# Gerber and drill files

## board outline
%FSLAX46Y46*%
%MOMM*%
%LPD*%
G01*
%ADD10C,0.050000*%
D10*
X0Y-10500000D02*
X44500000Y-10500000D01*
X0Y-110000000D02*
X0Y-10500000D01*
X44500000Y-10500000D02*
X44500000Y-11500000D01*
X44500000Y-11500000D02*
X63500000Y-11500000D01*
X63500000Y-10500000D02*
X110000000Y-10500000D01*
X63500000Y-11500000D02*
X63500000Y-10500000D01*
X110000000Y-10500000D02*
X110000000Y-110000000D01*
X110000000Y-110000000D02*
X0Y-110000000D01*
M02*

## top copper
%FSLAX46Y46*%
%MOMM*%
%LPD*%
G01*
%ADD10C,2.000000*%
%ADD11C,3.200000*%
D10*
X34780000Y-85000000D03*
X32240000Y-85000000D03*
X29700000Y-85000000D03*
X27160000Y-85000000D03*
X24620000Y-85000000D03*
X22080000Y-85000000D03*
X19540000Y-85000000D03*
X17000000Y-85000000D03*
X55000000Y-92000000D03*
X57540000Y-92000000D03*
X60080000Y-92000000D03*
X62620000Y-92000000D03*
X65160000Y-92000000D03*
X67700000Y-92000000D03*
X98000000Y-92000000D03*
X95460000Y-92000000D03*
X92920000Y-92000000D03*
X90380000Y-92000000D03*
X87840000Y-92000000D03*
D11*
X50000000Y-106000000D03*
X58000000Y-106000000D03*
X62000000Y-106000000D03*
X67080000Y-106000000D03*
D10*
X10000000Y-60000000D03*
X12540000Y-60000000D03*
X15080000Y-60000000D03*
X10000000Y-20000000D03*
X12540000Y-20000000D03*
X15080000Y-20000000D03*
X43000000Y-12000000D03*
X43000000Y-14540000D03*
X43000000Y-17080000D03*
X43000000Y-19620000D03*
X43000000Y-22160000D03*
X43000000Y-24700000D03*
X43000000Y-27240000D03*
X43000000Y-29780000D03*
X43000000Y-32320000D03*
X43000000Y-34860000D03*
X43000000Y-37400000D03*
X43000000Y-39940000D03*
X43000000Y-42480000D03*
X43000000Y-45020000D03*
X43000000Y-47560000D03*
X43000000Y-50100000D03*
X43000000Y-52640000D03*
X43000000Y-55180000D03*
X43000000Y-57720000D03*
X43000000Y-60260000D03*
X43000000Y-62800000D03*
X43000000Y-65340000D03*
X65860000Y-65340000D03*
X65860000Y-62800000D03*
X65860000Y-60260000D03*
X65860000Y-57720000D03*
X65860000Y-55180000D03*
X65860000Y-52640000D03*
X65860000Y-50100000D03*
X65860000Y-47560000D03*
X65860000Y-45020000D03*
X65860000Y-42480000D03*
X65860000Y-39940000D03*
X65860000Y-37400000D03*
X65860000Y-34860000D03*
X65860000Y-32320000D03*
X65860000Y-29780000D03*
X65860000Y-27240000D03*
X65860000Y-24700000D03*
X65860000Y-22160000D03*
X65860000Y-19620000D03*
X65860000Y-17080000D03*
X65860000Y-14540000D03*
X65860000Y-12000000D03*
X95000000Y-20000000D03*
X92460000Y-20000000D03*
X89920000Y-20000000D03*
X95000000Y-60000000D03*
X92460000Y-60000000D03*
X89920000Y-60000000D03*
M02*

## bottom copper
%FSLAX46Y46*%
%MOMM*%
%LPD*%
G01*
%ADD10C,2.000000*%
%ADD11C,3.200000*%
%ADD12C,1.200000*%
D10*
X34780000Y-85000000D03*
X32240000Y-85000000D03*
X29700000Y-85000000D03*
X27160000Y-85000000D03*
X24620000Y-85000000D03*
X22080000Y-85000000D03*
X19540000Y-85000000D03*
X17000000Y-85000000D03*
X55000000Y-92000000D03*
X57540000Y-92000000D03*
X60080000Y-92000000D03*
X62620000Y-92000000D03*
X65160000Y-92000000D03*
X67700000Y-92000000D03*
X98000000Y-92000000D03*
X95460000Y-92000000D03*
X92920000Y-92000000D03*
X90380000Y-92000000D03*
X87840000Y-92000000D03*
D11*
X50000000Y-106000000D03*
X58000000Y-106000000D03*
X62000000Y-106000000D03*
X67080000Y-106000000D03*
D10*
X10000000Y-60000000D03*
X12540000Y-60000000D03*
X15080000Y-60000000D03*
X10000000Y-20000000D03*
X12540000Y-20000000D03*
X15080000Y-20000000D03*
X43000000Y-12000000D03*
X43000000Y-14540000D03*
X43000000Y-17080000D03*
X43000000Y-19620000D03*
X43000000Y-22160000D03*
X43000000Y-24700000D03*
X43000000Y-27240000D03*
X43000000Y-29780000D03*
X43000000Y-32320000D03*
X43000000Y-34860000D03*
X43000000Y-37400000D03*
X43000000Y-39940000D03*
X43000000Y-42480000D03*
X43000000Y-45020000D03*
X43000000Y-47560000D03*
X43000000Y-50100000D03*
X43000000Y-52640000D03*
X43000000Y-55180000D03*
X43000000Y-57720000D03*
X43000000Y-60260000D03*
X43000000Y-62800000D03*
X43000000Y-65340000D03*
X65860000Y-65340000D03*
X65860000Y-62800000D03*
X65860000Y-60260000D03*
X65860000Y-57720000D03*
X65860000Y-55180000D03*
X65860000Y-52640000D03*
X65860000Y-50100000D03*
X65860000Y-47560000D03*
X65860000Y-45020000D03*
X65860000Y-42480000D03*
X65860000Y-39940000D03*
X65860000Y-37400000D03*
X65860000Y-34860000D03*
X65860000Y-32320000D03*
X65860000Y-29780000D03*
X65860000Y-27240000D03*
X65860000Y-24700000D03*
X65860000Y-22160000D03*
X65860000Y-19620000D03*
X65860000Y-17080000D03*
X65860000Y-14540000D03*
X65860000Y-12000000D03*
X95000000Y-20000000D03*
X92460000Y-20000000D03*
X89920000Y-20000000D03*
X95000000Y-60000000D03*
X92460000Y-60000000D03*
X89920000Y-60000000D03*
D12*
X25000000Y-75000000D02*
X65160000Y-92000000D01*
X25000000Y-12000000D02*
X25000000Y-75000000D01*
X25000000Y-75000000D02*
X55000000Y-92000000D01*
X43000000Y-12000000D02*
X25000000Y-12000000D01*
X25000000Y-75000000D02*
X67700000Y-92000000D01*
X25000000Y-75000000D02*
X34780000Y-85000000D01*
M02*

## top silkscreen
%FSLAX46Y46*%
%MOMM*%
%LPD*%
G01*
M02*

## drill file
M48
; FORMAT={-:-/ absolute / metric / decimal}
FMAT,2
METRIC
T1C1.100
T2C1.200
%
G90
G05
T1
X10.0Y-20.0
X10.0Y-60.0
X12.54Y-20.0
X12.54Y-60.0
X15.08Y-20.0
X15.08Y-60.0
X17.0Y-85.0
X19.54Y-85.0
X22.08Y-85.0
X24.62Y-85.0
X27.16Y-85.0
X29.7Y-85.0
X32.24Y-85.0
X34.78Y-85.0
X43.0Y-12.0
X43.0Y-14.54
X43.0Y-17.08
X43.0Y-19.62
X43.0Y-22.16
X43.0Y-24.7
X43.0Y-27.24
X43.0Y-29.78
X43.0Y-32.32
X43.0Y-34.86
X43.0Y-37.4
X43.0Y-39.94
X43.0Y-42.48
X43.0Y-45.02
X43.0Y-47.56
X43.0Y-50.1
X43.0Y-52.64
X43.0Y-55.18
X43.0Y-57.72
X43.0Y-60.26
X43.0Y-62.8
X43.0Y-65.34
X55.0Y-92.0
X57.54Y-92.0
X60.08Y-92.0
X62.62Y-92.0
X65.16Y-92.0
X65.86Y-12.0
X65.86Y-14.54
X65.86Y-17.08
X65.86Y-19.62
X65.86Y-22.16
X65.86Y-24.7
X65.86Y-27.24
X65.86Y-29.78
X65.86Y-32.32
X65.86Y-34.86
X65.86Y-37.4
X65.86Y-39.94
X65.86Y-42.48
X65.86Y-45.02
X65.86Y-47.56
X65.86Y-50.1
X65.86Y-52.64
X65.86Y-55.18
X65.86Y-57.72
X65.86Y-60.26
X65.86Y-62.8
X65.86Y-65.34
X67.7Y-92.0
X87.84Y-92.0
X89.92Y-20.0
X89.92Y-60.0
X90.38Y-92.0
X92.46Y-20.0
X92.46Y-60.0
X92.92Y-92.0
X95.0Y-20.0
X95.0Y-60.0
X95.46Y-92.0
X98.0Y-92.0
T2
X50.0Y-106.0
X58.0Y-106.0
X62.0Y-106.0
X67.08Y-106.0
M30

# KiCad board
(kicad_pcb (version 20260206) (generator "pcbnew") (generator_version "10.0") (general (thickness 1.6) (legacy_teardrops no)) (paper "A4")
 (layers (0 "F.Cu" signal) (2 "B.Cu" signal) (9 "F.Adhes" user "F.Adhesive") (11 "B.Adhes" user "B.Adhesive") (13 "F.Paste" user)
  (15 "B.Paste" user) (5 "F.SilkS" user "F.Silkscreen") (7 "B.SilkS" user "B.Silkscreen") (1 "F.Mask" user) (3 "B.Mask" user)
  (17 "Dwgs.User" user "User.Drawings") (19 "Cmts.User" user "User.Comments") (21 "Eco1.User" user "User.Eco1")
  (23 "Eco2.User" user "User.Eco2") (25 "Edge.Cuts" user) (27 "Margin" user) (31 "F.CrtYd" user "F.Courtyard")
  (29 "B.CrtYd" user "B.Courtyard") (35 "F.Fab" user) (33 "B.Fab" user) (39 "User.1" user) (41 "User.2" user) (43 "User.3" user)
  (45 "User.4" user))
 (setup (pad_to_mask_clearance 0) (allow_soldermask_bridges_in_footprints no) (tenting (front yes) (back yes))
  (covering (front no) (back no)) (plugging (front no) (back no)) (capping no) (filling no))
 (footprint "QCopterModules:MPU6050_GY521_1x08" (layer "F.Cu") (at 34.78 85 -90)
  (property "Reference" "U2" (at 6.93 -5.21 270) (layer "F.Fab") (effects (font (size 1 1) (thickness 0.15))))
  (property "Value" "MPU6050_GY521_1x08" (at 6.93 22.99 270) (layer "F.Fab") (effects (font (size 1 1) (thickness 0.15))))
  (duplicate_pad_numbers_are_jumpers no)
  (pad "1" thru_hole circle (at 0 0 270) (size 2 2) (drill 1.1) (layers "*.Cu" "*.Mask") (remove_unused_layers no) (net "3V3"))
  (pad "2" thru_hole circle (at 0 2.54 270) (size 2 2) (drill 1.1) (layers "*.Cu" "*.Mask") (remove_unused_layers no) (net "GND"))
  (pad "3" thru_hole circle (at 0 5.08 270) (size 2 2) (drill 1.1) (layers "*.Cu" "*.Mask") (remove_unused_layers no) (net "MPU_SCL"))
  (pad "4" thru_hole circle (at 0 7.62 270) (size 2 2) (drill 1.1) (layers "*.Cu" "*.Mask") (remove_unused_layers no) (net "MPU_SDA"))
  (pad "5" thru_hole circle (at 0 10.16 270) (size 2 2) (drill 1.1) (layers "*.Cu" "*.Mask") (remove_unused_layers no)
   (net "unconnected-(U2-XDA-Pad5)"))
  (pad "6" thru_hole circle (at 0 12.7 270) (size 2 2) (drill 1.1) (layers "*.Cu" "*.Mask") (remove_unused_layers no)
   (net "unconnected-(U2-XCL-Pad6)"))
  (pad "7" thru_hole circle (at 0 15.24 270) (size 2 2) (drill 1.1) (layers "*.Cu" "*.Mask") (remove_unused_layers no) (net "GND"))
  (pad "8" thru_hole circle (at 0 17.78 270) (size 2 2) (drill 1.1) (layers "*.Cu" "*.Mask") (remove_unused_layers no) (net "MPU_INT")))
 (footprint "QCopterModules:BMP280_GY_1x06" (layer "F.Cu") (at 55 92 90)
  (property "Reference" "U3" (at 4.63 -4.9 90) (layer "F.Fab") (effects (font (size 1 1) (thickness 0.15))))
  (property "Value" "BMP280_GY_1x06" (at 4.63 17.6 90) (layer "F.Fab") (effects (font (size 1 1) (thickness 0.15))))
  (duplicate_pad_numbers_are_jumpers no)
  (pad "1" thru_hole circle (at 0 0 90) (size 2 2) (drill 1.1) (layers "*.Cu" "*.Mask") (remove_unused_layers no) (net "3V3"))
  (pad "2" thru_hole circle (at 0 2.54 90) (size 2 2) (drill 1.1) (layers "*.Cu" "*.Mask") (remove_unused_layers no) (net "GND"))
  (pad "3" thru_hole circle (at 0 5.08 90) (size 2 2) (drill 1.1) (layers "*.Cu" "*.Mask") (remove_unused_layers no) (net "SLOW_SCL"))
  (pad "4" thru_hole circle (at 0 7.62 90) (size 2 2) (drill 1.1) (layers "*.Cu" "*.Mask") (remove_unused_layers no) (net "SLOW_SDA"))
  (pad "5" thru_hole circle (at 0 10.16 90) (size 2 2) (drill 1.1) (layers "*.Cu" "*.Mask") (remove_unused_layers no) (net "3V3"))
  (pad "6" thru_hole circle (at 0 12.7 90) (size 2 2) (drill 1.1) (layers "*.Cu" "*.Mask") (remove_unused_layers no) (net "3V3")))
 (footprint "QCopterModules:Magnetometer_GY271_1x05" (layer "F.Cu") (at 98 92 -90)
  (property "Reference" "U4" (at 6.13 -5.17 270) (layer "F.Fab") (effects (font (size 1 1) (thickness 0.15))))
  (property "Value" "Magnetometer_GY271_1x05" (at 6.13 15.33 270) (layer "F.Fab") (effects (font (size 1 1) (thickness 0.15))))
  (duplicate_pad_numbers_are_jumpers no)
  (pad "1" thru_hole circle (at 0 0 270) (size 2 2) (drill 1.1) (layers "*.Cu" "*.Mask") (remove_unused_layers no) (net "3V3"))
  (pad "2" thru_hole circle (at 0 2.54 270) (size 2 2) (drill 1.1) (layers "*.Cu" "*.Mask") (remove_unused_layers no) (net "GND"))
  (pad "3" thru_hole circle (at 0 5.08 270) (size 2 2) (drill 1.1) (layers "*.Cu" "*.Mask") (remove_unused_layers no) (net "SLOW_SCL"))
  (pad "4" thru_hole circle (at 0 7.62 270) (size 2 2) (drill 1.1) (layers "*.Cu" "*.Mask") (remove_unused_layers no) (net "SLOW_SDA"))
  (pad "5" thru_hole circle (at 0 10.16 270) (size 2 2) (drill 1.1) (layers "*.Cu" "*.Mask") (remove_unused_layers no) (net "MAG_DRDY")))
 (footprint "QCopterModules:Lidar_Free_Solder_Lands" (layer "F.Cu") (at 50 106)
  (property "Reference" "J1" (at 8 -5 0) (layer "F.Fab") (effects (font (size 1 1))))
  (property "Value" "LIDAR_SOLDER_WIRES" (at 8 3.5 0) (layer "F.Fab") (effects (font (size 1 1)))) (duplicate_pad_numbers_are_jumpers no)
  (pad "1" thru_hole circle (at 0 0) (size 3.2 3.2) (drill 1.2) (layers "*.Cu" "*.Mask") (remove_unused_layers no) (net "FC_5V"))
  (pad "2" thru_hole circle (at 8 0) (size 3.2 3.2) (drill 1.2) (layers "*.Cu" "*.Mask") (remove_unused_layers no) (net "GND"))
  (pad "3" thru_hole circle (at 12 0) (size 3.2 3.2) (drill 1.2) (layers "*.Cu" "*.Mask") (remove_unused_layers no) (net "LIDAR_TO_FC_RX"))
  (pad "4" thru_hole circle (at 17.08 0) (size 3.2 3.2) (drill 1.2) (layers "*.Cu" "*.Mask") (remove_unused_layers no)
   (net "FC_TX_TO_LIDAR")))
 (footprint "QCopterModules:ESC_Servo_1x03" (layer "F.Cu") (at 10 60 90)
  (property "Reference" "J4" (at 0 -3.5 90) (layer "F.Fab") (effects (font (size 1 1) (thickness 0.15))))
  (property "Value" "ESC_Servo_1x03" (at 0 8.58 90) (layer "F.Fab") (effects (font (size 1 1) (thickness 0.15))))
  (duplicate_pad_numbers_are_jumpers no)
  (pad "1" thru_hole circle (at 0 0 90) (size 2 2) (drill 1.1) (layers "*.Cu" "*.Mask") (remove_unused_layers no) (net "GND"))
  (pad "2" thru_hole circle (at 0 2.54 90) (size 2 2) (drill 1.1) (layers "*.Cu" "*.Mask") (remove_unused_layers no) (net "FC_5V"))
  (pad "3" thru_hole circle (at 0 5.08 90) (size 2 2) (drill 1.1) (layers "*.Cu" "*.Mask") (remove_unused_layers no) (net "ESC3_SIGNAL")))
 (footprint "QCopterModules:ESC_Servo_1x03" (layer "F.Cu") (at 10 20 90)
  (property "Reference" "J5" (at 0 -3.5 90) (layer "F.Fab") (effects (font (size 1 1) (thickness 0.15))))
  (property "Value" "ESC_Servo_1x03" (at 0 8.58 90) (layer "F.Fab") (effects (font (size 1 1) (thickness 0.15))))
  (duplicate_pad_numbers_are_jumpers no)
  (pad "1" thru_hole circle (at 0 0 90) (size 2 2) (drill 1.1) (layers "*.Cu" "*.Mask") (remove_unused_layers no) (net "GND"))
  (pad "2" thru_hole circle (at 0 2.54 90) (size 2 2) (drill 1.1) (layers "*.Cu" "*.Mask") (remove_unused_layers no)
   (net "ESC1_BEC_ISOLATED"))
  (pad "3" thru_hole circle (at 0 5.08 90) (size 2 2) (drill 1.1) (layers "*.Cu" "*.Mask") (remove_unused_layers no) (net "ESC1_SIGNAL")))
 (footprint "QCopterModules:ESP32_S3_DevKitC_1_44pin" (layer "F.Cu") (at 43 12)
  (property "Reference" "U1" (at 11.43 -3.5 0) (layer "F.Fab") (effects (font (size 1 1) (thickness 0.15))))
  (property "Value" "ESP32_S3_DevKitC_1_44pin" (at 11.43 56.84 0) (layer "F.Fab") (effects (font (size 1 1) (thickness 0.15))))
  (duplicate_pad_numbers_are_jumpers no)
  (pad "1" thru_hole circle (at 0 0) (size 2 2) (drill 1.1) (layers "*.Cu" "*.Mask") (remove_unused_layers no) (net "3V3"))
  (pad "2" thru_hole circle (at 0 2.54) (size 2 2) (drill 1.1) (layers "*.Cu" "*.Mask") (remove_unused_layers no))
  (pad "3" thru_hole circle (at 0 5.08) (size 2 2) (drill 1.1) (layers "*.Cu" "*.Mask") (remove_unused_layers no)
   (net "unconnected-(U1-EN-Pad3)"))
  (pad "4" thru_hole circle (at 0 7.62) (size 2 2) (drill 1.1) (layers "*.Cu" "*.Mask") (remove_unused_layers no) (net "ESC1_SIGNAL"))
  (pad "5" thru_hole circle (at 0 10.16) (size 2 2) (drill 1.1) (layers "*.Cu" "*.Mask") (remove_unused_layers no)
   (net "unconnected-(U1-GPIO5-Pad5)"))
  (pad "6" thru_hole circle (at 0 12.7) (size 2 2) (drill 1.1) (layers "*.Cu" "*.Mask") (remove_unused_layers no)
   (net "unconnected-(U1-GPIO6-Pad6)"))
  (pad "7" thru_hole circle (at 0 15.24) (size 2 2) (drill 1.1) (layers "*.Cu" "*.Mask") (remove_unused_layers no)
   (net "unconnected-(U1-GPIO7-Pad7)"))
  (pad "8" thru_hole circle (at 0 17.78) (size 2 2) (drill 1.1) (layers "*.Cu" "*.Mask") (remove_unused_layers no) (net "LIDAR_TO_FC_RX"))
  (pad "9" thru_hole circle (at 0 20.32) (size 2 2) (drill 1.1) (layers "*.Cu" "*.Mask") (remove_unused_layers no) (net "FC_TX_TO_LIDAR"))
  (pad "10" thru_hole circle (at 0 22.86) (size 2 2) (drill 1.1) (layers "*.Cu" "*.Mask") (remove_unused_layers no)
   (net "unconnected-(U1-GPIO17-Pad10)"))
  (pad "11" thru_hole circle (at 0 25.4) (size 2 2) (drill 1.1) (layers "*.Cu" "*.Mask") (remove_unused_layers no) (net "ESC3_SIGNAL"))
  (pad "12" thru_hole circle (at 0 27.94) (size 2 2) (drill 1.1) (layers "*.Cu" "*.Mask") (remove_unused_layers no)
   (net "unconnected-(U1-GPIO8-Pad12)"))
  (pad "13" thru_hole circle (at 0 30.48) (size 2 2) (drill 1.1) (layers "*.Cu" "*.Mask") (remove_unused_layers no)
   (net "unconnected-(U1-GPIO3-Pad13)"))
  (pad "14" thru_hole circle (at 0 33.02) (size 2 2) (drill 1.1) (layers "*.Cu" "*.Mask") (remove_unused_layers no)
   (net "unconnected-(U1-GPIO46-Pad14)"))
  (pad "15" thru_hole circle (at 0 35.56) (size 2 2) (drill 1.1) (layers "*.Cu" "*.Mask") (remove_unused_layers no)
   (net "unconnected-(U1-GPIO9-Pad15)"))
  (pad "16" thru_hole circle (at 0 38.1) (size 2 2) (drill 1.1) (layers "*.Cu" "*.Mask") (remove_unused_layers no)
   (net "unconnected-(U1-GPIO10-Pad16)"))
  (pad "17" thru_hole circle (at 0 40.64) (size 2 2) (drill 1.1) (layers "*.Cu" "*.Mask") (remove_unused_layers no)
   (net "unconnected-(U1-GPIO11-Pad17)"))
  (pad "18" thru_hole circle (at 0 43.18) (size 2 2) (drill 1.1) (layers "*.Cu" "*.Mask") (remove_unused_layers no) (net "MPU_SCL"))
  (pad "19" thru_hole circle (at 0 45.72) (size 2 2) (drill 1.1) (layers "*.Cu" "*.Mask") (remove_unused_layers no) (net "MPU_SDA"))
  (pad "20" thru_hole circle (at 0 48.26) (size 2 2) (drill 1.1) (layers "*.Cu" "*.Mask") (remove_unused_layers no) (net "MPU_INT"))
  (pad "21" thru_hole circle (at 0 50.8) (size 2 2) (drill 1.1) (layers "*.Cu" "*.Mask") (remove_unused_layers no) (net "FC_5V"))
  (pad "22" thru_hole circle (at 0 53.34) (size 2 2) (drill 1.1) (layers "*.Cu" "*.Mask") (remove_unused_layers no) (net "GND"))
  (pad "23" thru_hole circle (at 22.86 53.34) (size 2 2) (drill 1.1) (layers "*.Cu" "*.Mask") (remove_unused_layers no) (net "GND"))
  (pad "24" thru_hole circle (at 22.86 50.8) (size 2 2) (drill 1.1) (layers "*.Cu" "*.Mask") (remove_unused_layers no) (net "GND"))
  (pad "25" thru_hole circle (at 22.86 48.26) (size 2 2) (drill 1.1) (layers "*.Cu" "*.Mask") (remove_unused_layers no)
   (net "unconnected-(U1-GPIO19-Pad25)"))
  (pad "26" thru_hole circle (at 22.86 45.72) (size 2 2) (drill 1.1) (layers "*.Cu" "*.Mask") (remove_unused_layers no)
   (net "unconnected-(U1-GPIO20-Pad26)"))
  (pad "27" thru_hole circle (at 22.86 43.18) (size 2 2) (drill 1.1) (layers "*.Cu" "*.Mask") (remove_unused_layers no) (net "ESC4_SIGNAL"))
  (pad "28" thru_hole circle (at 22.86 40.64) (size 2 2) (drill 1.1) (layers "*.Cu" "*.Mask") (remove_unused_layers no)
   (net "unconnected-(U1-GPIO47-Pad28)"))
  (pad "29" thru_hole circle (at 22.86 38.1) (size 2 2) (drill 1.1) (layers "*.Cu" "*.Mask") (remove_unused_layers no)
   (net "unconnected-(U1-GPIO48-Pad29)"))
  (pad "30" thru_hole circle (at 22.86 35.56) (size 2 2) (drill 1.1) (layers "*.Cu" "*.Mask") (remove_unused_layers no)
   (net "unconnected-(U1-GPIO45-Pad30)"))
  (pad "31" thru_hole circle (at 22.86 33.02) (size 2 2) (drill 1.1) (layers "*.Cu" "*.Mask") (remove_unused_layers no)
   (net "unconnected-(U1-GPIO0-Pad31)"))
  (pad "32" thru_hole circle (at 22.86 30.48) (size 2 2) (drill 1.1) (layers "*.Cu" "*.Mask") (remove_unused_layers no)
   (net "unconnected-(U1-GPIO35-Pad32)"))
  (pad "33" thru_hole circle (at 22.86 27.94) (size 2 2) (drill 1.1) (layers "*.Cu" "*.Mask") (remove_unused_layers no)
   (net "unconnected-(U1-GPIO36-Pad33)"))
  (pad "34" thru_hole circle (at 22.86 25.4) (size 2 2) (drill 1.1) (layers "*.Cu" "*.Mask") (remove_unused_layers no)
   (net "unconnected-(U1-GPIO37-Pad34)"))
  (pad "35" thru_hole circle (at 22.86 22.86) (size 2 2) (drill 1.1) (layers "*.Cu" "*.Mask") (remove_unused_layers no)
   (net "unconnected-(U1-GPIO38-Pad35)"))
  (pad "36" thru_hole circle (at 22.86 20.32) (size 2 2) (drill 1.1) (layers "*.Cu" "*.Mask") (remove_unused_layers no) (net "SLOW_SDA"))
  (pad "37" thru_hole circle (at 22.86 17.78) (size 2 2) (drill 1.1) (layers "*.Cu" "*.Mask") (remove_unused_layers no) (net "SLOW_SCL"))
  (pad "38" thru_hole circle (at 22.86 15.24) (size 2 2) (drill 1.1) (layers "*.Cu" "*.Mask") (remove_unused_layers no) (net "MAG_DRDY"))
  (pad "39" thru_hole circle (at 22.86 12.7) (size 2 2) (drill 1.1) (layers "*.Cu" "*.Mask") (remove_unused_layers no)
   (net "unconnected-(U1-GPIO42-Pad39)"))
  (pad "40" thru_hole circle (at 22.86 10.16) (size 2 2) (drill 1.1) (layers "*.Cu" "*.Mask") (remove_unused_layers no) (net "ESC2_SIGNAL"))
  (pad "41" thru_hole circle (at 22.86 7.62) (size 2 2) (drill 1.1) (layers "*.Cu" "*.Mask") (remove_unused_layers no)
   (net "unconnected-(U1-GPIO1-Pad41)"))
  (pad "42" thru_hole circle (at 22.86 5.08) (size 2 2) (drill 1.1) (layers "*.Cu" "*.Mask") (remove_unused_layers no)
   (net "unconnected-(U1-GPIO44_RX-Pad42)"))
  (pad "43" thru_hole circle (at 22.86 2.54) (size 2 2) (drill 1.1) (layers "*.Cu" "*.Mask") (remove_unused_layers no)
   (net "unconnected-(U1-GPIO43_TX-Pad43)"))
  (pad "44" thru_hole circle (at 22.86 0) (size 2 2) (drill 1.1) (layers "*.Cu" "*.Mask") (remove_unused_layers no) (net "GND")))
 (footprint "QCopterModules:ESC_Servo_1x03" (layer "F.Cu") (at 95 20 -90)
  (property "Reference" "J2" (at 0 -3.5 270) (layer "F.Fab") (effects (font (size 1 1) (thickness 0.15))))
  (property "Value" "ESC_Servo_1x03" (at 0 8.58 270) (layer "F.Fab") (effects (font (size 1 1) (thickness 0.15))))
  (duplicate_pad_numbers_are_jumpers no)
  (pad "1" thru_hole circle (at 0 0 270) (size 2 2) (drill 1.1) (layers "*.Cu" "*.Mask") (remove_unused_layers no) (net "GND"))
  (pad "2" thru_hole circle (at 0 2.54 270) (size 2 2) (drill 1.1) (layers "*.Cu" "*.Mask") (remove_unused_layers no)
   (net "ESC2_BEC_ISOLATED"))
  (pad "3" thru_hole circle (at 0 5.08 270) (size 2 2) (drill 1.1) (layers "*.Cu" "*.Mask") (remove_unused_layers no) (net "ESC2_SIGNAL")))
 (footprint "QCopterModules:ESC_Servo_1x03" (layer "F.Cu") (at 95 60 -90)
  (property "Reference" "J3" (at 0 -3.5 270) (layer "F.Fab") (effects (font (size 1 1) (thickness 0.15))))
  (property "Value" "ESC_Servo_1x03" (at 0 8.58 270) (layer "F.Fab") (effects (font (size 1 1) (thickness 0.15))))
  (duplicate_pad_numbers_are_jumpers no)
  (pad "1" thru_hole circle (at 0 0 270) (size 2 2) (drill 1.1) (layers "*.Cu" "*.Mask") (remove_unused_layers no) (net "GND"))
  (pad "2" thru_hole circle (at 0 2.54 270) (size 2 2) (drill 1.1) (layers "*.Cu" "*.Mask") (remove_unused_layers no)
   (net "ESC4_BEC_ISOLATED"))
  (pad "3" thru_hole circle (at 0 5.08 270) (size 2 2) (drill 1.1) (layers "*.Cu" "*.Mask") (remove_unused_layers no) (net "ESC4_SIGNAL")))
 (gr_line (start 0 10.5) (end 44.5 10.5) (stroke (width 0.05) (type default)) (layer "Edge.Cuts"))
 (gr_line (start 0 110) (end 0 10.5) (stroke (width 0.05) (type default)) (layer "Edge.Cuts"))
 (gr_line (start 44.5 10.5) (end 44.5 11.5) (stroke (width 0.05) (type default)) (layer "Edge.Cuts"))
 (gr_line (start 44.5 11.5) (end 63.5 11.5) (stroke (width 0.05) (type default)) (layer "Edge.Cuts"))
 (gr_line (start 63.5 10.5) (end 110 10.5) (stroke (width 0.05) (type default)) (layer "Edge.Cuts"))
 (gr_line (start 63.5 11.5) (end 63.5 10.5) (stroke (width 0.05) (type default)) (layer "Edge.Cuts"))
 (gr_line (start 110 10.5) (end 110 110) (stroke (width 0.05) (type default)) (layer "Edge.Cuts"))
 (gr_line (start 110 110) (end 0 110) (stroke (width 0.05) (type default)) (layer "Edge.Cuts"))
 (segment (start 25 75) (end 65.16 92) (width 1.2) (layer "B.Cu") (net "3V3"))
 (segment (start 25 12) (end 25 75) (width 1.2) (layer "B.Cu") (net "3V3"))
 (segment (start 25 75) (end 55 92) (width 1.2) (layer "B.Cu") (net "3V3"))
 (segment (start 43 12) (end 25 12) (width 1.2) (layer "B.Cu") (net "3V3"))
 (segment (start 25 75) (end 67.7 92) (width 1.2) (layer "B.Cu") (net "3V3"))
 (segment (start 25 75) (end 34.78 85) (width 1.2) (layer "B.Cu") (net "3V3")))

